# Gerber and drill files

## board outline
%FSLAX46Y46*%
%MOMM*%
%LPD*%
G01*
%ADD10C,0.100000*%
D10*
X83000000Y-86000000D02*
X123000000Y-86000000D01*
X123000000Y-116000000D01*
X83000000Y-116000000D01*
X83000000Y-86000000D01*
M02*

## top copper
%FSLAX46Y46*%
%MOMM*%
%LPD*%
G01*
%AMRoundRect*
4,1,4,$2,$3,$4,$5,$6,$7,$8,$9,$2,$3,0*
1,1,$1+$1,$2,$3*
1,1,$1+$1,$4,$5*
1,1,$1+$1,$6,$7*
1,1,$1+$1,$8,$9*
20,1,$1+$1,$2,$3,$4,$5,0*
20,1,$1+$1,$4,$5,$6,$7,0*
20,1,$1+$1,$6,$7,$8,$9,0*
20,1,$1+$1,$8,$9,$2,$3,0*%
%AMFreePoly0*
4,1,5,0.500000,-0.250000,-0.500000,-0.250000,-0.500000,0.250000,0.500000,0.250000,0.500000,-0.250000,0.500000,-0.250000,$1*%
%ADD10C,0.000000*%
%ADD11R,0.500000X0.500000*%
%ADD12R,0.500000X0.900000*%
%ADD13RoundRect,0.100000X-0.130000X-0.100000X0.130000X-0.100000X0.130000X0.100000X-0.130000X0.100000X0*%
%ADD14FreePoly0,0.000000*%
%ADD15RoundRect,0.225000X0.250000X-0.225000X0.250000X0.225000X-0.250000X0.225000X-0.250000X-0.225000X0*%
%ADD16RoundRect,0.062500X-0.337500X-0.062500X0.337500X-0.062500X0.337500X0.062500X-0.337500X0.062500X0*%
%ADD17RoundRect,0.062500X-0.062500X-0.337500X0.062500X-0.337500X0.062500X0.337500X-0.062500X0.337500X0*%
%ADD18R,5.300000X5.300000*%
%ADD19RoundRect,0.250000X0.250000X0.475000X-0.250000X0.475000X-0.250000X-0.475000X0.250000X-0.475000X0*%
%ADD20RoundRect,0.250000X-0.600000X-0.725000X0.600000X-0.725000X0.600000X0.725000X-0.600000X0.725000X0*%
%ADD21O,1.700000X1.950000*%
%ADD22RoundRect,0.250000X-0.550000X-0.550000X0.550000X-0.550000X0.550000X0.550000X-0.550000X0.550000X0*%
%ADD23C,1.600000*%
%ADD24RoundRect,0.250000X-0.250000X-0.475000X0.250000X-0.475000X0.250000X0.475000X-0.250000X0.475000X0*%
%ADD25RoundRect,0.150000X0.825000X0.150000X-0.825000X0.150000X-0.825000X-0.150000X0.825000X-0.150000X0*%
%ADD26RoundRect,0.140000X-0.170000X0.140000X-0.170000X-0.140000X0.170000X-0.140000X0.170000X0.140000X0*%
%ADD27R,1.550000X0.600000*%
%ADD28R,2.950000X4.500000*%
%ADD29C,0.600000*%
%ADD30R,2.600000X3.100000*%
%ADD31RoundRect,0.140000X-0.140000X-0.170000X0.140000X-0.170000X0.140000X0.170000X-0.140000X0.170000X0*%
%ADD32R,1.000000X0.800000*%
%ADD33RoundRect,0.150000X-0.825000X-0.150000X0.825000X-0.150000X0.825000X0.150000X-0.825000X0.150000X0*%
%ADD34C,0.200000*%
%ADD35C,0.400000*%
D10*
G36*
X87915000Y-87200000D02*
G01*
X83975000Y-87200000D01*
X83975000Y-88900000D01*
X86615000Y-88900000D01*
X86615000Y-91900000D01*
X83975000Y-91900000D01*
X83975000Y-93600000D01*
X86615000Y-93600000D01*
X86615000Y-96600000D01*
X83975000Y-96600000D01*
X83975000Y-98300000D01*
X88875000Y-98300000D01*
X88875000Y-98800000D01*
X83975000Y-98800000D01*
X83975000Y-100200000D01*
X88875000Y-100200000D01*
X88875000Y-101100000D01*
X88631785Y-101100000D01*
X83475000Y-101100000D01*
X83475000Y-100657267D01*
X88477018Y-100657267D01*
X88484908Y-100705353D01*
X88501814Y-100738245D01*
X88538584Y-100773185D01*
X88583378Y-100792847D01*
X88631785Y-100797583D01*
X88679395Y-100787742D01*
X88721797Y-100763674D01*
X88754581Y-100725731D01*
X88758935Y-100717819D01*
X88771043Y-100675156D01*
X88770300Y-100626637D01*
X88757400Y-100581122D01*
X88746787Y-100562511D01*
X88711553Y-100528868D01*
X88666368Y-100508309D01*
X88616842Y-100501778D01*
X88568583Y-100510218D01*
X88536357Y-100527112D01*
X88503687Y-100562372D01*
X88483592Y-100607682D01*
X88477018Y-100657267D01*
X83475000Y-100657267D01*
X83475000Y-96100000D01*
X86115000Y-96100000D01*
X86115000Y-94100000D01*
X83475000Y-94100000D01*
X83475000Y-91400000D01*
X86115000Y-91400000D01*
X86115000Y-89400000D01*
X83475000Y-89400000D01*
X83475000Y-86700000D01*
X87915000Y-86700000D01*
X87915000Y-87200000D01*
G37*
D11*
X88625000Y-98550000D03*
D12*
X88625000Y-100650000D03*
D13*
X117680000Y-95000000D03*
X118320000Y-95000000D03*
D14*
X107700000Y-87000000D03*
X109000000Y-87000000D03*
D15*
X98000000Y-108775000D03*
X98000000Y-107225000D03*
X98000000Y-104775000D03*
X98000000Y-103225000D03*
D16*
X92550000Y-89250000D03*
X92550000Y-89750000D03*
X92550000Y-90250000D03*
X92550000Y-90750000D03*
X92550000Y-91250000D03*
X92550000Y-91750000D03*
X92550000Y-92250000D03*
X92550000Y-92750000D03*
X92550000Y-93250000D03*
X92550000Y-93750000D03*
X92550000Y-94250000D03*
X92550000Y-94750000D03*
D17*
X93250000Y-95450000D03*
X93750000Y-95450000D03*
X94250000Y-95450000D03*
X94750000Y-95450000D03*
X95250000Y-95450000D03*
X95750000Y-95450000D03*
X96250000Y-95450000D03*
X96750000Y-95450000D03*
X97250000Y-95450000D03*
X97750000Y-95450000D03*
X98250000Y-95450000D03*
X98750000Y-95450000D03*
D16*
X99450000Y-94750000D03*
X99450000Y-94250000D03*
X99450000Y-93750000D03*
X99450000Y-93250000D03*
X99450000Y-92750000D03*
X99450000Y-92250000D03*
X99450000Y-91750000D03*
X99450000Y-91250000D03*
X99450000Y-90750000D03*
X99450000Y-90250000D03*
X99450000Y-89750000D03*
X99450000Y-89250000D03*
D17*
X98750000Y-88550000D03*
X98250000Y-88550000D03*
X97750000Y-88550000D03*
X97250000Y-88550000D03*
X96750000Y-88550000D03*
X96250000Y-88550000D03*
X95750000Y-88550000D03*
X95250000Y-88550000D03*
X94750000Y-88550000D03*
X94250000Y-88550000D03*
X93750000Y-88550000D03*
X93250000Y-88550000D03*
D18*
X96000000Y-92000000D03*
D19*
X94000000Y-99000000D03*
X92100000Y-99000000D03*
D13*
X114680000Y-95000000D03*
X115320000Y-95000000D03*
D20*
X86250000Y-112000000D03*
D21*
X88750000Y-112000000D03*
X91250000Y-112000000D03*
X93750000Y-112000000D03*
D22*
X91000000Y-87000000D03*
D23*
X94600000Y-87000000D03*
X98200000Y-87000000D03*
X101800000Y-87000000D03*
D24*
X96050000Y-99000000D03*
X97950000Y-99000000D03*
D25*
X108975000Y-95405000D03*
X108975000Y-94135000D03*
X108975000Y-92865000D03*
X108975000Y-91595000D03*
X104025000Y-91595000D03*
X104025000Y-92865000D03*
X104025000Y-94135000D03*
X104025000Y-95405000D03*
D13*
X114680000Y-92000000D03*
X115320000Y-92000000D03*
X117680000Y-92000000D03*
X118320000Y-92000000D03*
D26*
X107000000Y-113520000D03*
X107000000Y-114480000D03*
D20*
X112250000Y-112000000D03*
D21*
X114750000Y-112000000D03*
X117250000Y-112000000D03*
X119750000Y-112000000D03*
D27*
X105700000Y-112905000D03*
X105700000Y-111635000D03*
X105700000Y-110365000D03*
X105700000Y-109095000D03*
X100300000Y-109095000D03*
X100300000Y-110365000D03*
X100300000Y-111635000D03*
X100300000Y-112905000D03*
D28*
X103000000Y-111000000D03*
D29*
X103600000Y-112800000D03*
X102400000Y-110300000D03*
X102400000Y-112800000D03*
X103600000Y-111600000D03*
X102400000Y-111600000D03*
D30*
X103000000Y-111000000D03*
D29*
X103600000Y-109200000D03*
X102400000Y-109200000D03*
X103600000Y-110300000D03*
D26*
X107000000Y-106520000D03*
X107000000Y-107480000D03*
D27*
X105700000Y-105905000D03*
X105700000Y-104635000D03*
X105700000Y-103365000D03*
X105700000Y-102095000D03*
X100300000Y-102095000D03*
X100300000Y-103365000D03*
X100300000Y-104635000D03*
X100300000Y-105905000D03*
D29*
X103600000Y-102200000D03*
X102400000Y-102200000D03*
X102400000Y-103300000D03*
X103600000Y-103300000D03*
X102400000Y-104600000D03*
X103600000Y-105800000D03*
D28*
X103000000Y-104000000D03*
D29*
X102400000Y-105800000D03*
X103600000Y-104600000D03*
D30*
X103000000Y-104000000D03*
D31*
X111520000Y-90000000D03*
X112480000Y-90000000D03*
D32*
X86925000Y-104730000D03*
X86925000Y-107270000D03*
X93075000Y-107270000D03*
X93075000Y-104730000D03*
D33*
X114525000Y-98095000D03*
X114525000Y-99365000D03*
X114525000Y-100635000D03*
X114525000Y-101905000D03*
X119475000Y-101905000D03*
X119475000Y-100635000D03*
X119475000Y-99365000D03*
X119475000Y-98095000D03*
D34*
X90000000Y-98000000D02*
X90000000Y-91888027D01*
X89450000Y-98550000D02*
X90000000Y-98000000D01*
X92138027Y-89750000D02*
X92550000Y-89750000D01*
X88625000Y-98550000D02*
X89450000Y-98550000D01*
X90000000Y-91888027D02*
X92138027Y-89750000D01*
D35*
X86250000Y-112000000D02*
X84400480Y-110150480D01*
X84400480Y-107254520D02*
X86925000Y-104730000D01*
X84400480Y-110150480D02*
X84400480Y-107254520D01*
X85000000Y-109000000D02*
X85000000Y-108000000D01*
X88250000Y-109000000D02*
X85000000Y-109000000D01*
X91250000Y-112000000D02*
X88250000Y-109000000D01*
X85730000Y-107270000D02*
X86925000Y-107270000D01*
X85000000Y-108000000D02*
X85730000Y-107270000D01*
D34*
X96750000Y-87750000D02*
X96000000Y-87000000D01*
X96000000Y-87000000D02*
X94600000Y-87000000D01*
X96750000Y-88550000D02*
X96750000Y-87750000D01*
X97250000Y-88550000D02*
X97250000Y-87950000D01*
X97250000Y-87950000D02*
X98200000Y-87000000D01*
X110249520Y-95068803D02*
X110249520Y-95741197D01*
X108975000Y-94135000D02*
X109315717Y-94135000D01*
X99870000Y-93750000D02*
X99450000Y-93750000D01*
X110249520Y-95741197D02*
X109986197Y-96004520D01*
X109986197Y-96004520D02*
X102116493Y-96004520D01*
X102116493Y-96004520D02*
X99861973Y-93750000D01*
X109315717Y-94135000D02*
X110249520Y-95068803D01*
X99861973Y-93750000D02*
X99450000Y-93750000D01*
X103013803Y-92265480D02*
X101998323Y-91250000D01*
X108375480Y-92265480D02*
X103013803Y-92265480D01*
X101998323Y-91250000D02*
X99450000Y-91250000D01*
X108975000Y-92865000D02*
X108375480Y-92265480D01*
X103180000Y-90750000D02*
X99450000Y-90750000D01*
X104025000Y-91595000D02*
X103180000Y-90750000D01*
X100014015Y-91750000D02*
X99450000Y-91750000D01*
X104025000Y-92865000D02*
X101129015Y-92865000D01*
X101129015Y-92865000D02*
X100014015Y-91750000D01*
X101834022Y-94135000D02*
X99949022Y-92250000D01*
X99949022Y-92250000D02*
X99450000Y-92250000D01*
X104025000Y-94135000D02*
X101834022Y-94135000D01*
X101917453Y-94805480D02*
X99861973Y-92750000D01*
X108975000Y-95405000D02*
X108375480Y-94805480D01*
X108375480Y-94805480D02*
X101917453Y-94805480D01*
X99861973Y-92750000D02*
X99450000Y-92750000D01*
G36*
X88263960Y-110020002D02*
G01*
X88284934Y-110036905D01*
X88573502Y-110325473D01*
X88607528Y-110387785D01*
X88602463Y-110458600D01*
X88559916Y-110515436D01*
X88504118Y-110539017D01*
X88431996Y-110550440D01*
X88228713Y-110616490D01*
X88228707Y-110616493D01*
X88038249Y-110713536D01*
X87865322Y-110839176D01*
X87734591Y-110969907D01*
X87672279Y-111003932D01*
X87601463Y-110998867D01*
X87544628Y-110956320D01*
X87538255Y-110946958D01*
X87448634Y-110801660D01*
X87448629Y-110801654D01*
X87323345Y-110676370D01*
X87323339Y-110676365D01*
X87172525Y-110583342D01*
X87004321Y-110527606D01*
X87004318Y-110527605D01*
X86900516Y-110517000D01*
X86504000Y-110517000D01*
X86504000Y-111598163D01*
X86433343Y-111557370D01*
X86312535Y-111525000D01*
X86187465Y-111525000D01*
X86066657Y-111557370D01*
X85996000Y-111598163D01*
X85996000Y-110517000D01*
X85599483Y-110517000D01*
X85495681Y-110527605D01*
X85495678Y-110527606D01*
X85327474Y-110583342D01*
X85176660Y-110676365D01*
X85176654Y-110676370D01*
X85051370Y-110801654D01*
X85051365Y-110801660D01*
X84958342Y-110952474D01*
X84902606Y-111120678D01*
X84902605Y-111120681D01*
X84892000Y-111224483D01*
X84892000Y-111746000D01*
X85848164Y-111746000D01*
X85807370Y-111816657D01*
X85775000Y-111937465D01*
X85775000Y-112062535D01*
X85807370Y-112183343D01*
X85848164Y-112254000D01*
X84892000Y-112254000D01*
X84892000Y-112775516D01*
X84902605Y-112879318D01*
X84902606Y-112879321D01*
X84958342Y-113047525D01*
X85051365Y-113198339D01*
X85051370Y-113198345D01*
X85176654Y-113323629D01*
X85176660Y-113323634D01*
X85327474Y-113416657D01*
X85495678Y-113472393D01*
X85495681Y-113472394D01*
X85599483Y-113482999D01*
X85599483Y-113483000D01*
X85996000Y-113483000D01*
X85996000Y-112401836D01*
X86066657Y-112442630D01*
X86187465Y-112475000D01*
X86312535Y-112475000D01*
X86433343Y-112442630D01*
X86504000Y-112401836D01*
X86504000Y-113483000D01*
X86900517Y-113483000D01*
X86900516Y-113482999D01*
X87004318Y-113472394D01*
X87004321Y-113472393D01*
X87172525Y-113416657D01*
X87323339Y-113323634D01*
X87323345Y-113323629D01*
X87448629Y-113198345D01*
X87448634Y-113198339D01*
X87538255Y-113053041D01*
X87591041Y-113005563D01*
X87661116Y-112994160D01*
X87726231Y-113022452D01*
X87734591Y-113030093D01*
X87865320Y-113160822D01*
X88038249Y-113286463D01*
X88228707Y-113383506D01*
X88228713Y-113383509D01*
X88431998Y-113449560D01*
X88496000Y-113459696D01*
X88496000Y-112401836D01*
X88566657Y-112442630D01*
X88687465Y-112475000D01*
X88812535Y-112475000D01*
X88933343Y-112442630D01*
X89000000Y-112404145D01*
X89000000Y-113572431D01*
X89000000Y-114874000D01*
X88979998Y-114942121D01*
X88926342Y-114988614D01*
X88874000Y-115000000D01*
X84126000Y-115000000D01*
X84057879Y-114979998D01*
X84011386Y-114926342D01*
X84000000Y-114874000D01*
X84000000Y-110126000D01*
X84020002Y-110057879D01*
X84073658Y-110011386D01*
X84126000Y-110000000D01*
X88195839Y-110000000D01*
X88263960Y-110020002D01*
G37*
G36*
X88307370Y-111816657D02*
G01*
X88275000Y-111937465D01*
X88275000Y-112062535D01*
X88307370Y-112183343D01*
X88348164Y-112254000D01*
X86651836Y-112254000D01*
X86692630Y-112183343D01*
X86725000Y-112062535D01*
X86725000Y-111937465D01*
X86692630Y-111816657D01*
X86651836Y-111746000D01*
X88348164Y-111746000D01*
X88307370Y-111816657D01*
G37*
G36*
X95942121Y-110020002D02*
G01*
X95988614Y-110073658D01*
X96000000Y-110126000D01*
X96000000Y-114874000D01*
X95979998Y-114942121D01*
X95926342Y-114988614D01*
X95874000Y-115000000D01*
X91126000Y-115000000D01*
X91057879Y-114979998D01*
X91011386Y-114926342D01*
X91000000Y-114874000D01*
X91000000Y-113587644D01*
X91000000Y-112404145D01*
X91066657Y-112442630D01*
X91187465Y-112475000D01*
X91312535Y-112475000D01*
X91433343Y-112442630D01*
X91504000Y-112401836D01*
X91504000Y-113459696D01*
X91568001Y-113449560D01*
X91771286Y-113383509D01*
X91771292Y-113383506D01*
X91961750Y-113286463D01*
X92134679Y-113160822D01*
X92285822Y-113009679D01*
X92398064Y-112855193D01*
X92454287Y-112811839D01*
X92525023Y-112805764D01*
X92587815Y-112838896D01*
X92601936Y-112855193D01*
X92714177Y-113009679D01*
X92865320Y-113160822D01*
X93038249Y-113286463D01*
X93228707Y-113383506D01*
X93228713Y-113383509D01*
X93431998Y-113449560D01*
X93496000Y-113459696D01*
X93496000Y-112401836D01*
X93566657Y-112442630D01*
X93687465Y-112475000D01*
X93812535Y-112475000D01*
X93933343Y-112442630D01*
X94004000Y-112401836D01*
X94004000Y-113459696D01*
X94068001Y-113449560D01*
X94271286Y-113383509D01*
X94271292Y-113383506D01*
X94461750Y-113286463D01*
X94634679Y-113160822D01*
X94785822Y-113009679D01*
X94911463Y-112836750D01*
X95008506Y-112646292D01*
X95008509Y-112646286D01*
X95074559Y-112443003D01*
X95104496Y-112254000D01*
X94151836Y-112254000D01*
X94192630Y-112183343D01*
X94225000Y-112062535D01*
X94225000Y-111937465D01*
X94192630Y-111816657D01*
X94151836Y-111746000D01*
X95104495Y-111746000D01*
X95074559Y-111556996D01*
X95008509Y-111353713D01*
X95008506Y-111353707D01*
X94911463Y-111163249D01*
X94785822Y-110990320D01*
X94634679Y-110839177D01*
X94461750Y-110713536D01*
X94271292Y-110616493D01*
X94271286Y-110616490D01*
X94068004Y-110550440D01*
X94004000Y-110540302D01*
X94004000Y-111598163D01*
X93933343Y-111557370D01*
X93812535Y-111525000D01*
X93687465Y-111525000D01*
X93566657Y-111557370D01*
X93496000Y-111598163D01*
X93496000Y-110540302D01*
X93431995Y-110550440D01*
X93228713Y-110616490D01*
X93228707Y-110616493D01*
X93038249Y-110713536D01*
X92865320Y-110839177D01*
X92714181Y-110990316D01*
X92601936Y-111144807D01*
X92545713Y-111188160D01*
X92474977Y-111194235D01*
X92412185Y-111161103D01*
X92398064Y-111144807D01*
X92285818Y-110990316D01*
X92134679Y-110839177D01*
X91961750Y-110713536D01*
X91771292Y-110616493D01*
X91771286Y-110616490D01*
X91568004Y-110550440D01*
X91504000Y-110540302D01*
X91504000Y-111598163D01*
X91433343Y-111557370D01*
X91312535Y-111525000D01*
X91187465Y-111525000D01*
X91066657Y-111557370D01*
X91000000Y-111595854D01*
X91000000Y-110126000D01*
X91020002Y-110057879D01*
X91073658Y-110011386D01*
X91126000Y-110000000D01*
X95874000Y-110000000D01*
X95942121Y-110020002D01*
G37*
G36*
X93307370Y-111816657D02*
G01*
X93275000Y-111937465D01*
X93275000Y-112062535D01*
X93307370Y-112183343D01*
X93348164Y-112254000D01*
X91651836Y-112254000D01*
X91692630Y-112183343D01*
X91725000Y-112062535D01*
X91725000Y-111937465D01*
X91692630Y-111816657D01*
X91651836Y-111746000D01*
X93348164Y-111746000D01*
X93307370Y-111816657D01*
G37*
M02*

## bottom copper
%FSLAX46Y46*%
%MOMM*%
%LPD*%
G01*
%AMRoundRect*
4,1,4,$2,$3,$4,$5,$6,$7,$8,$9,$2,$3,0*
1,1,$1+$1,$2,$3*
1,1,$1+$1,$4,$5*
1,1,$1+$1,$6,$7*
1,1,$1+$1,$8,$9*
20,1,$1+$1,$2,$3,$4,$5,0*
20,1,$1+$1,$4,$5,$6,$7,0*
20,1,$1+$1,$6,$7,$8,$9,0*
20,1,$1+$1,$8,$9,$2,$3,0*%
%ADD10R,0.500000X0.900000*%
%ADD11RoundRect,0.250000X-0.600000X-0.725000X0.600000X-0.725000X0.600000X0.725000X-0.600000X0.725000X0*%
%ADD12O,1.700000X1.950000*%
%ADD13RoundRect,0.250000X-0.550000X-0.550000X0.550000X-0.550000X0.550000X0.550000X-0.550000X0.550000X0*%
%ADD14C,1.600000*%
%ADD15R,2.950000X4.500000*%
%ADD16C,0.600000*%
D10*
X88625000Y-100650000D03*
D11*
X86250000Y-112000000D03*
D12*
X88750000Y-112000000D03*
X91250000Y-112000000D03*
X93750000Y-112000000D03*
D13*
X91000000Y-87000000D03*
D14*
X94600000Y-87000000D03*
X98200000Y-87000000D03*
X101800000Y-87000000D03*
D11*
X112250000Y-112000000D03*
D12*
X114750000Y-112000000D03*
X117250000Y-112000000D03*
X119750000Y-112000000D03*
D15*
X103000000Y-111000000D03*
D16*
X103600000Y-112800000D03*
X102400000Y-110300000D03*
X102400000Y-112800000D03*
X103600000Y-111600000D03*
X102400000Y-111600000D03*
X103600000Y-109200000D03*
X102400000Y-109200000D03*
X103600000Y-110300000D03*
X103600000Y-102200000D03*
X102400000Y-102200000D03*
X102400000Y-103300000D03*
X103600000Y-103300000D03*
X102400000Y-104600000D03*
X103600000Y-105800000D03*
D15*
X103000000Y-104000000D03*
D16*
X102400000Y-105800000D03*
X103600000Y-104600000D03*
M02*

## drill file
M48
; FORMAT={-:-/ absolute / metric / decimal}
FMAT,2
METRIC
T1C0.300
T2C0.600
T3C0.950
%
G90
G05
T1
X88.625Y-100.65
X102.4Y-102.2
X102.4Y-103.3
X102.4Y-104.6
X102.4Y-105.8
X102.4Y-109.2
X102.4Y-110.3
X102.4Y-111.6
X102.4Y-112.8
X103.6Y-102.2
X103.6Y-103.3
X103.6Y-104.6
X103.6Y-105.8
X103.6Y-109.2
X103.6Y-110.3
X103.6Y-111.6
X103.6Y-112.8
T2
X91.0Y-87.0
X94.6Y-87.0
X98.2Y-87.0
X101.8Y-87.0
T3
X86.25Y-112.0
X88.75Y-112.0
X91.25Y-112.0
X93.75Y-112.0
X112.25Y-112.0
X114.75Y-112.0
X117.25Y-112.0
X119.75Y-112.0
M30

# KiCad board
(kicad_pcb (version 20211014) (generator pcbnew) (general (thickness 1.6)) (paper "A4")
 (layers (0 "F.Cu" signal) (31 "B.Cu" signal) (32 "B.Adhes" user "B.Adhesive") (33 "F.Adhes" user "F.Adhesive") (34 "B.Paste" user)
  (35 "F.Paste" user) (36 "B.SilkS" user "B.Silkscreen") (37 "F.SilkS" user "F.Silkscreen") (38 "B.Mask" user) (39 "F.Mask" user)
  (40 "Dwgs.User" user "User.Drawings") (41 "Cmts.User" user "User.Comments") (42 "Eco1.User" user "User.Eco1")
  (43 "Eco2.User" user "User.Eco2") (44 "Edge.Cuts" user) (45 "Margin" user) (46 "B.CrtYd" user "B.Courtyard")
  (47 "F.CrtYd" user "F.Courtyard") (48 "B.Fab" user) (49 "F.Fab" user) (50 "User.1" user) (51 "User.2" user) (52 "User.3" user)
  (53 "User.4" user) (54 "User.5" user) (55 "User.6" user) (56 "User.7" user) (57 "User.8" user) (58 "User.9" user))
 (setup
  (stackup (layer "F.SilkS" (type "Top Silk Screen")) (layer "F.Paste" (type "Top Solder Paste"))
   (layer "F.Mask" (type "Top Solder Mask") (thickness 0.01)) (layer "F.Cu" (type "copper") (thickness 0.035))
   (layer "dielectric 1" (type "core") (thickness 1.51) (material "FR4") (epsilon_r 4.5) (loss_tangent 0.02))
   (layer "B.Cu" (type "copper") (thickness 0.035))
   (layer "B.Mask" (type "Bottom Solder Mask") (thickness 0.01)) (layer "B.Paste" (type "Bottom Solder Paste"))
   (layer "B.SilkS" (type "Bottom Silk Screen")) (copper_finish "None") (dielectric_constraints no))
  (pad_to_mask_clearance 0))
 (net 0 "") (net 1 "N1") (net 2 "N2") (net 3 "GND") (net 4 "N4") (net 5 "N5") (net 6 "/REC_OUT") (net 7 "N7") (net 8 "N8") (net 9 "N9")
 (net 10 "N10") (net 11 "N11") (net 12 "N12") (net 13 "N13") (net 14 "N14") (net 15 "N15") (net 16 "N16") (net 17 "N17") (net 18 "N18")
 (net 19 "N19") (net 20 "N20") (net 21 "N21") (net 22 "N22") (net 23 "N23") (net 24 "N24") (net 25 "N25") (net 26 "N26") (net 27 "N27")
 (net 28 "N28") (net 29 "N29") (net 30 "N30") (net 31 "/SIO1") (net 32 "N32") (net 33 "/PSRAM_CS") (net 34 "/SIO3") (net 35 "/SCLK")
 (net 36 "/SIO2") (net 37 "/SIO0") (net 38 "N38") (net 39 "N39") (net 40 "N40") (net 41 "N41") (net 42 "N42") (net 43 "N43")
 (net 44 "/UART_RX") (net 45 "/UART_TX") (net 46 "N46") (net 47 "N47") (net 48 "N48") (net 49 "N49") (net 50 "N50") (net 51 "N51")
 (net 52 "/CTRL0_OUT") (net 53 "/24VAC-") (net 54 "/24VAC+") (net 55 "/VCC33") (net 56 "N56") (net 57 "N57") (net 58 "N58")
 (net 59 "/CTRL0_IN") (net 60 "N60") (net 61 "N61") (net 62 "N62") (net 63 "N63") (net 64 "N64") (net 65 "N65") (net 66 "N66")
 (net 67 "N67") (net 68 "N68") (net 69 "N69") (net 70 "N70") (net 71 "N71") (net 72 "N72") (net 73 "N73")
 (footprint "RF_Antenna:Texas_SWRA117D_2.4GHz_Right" (layer "F.Cu") (at 88.625 98.55 90)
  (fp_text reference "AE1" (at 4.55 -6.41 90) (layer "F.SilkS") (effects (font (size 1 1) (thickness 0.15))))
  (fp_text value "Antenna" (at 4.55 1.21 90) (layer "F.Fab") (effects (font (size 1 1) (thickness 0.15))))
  (fp_poly
   (pts (xy 2.45 -2.51) (xy 4.45 -2.51) (xy 4.45 -5.15) (xy 7.15 -5.15) (xy 7.15 -2.51) (xy 9.15 -2.51) (xy 9.15 -5.15) (xy 11.85 -5.15)
    (xy 11.85 -0.71) (xy 11.35 -0.71) (xy 11.35 -4.65) (xy 9.65 -4.65) (xy 9.65 -2.01) (xy 6.65 -2.01) (xy 6.65 -4.65) (xy 4.95 -4.65)
    (xy 4.95 -2.01) (xy 1.95 -2.01) (xy 1.95 -4.65) (xy 0.25 -4.65) (xy 0.25 0.25) (xy -0.25 0.25) (xy -0.25 -4.65) (xy -1.65 -4.65)
    (xy -1.65 0.25) (xy -2.55 0.25) (xy -2.55 0.006785) (xy -2.247583 0.006785) (xy -2.237742 0.054395) (xy -2.213674 0.096797)
    (xy -2.175731 0.129581) (xy -2.167819 0.133935) (xy -2.125156 0.146043) (xy -2.076637 0.1453) (xy -2.031122 0.1324)
    (xy -2.012511 0.121787) (xy -1.978868 0.086553) (xy -1.958309 0.041368) (xy -1.951778 -0.008158) (xy -1.960218 -0.056417)
    (xy -1.977112 -0.088643) (xy -2.012372 -0.121313) (xy -2.057682 -0.141408) (xy -2.107267 -0.147982) (xy -2.155353 -0.140092)
    (xy -2.188245 -0.123186) (xy -2.223185 -0.086416) (xy -2.242847 -0.041622) (xy -2.247583 0.006785) (xy -2.55 0.006785) (xy -2.55 -5.15)
    (xy 2.45 -5.15) (xy 2.45 -2.51))
   (layer "F.Cu") (width 0) (fill solid))
  (pad "1" connect rect (at 0 0 90) (size 0.5 0.5) (layers "F.Cu") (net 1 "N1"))
  (pad "2" thru_hole rect (at -2.1 0 90) (size 0.9 0.5) (drill 0.3) (layers *.Cu) (zone_connect 2)))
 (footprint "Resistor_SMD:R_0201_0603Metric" (layer "F.Cu") (at 118 95)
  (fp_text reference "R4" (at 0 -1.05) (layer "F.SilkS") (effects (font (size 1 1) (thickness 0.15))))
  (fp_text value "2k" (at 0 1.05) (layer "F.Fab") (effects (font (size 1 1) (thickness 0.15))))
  (pad "" smd roundrect (at 0.345 0) (size 0.318 0.36) (layers "F.Paste") (roundrect_rratio 0.25))
  (pad "" smd roundrect (at -0.345 0) (size 0.318 0.36) (layers "F.Paste") (roundrect_rratio 0.25))
  (pad "1" smd roundrect (at -0.32 0) (size 0.46 0.4) (layers "F.Cu" "F.Mask") (roundrect_rratio 0.25) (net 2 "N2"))
  (pad "2" smd roundrect (at 0.32 0) (size 0.46 0.4) (layers "F.Cu" "F.Mask") (roundrect_rratio 0.25) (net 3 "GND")))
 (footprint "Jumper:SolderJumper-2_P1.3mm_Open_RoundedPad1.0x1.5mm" (layer "F.Cu") (at 108.35 87)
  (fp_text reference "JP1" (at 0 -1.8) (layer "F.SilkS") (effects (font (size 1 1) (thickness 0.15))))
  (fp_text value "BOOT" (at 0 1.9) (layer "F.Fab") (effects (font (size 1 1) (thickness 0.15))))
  (pad "1" smd custom (at -0.65 0) (size 1 0.5) (layers "F.Cu" "F.Mask") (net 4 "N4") (zone_connect 2)
   (options (clearance outline) (anchor rect)) (primitives))
  (pad "2" smd custom (at 0.65 0) (size 1 0.5) (layers "F.Cu" "F.Mask") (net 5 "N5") (zone_connect 2)
   (options (clearance outline) (anchor rect)) (primitives)))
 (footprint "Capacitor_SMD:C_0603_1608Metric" (layer "F.Cu") (at 98 108 90)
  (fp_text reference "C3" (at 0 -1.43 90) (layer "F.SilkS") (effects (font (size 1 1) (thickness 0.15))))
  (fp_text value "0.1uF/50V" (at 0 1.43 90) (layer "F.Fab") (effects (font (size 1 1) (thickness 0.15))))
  (pad "1" smd roundrect (at -0.775 0 90) (size 0.9 0.95) (layers "F.Cu" "F.Paste" "F.Mask") (roundrect_rratio 0.25) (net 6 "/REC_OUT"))
  (pad "2" smd roundrect (at 0.775 0 90) (size 0.9 0.95) (layers "F.Cu" "F.Paste" "F.Mask") (roundrect_rratio 0.25) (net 3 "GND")))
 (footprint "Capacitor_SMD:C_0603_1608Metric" (layer "F.Cu") (at 98 104 90)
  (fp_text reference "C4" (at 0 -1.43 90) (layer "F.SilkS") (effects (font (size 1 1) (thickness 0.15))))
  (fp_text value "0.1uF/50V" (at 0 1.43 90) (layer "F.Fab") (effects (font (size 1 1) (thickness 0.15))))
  (pad "1" smd roundrect (at -0.775 0 90) (size 0.9 0.95) (layers "F.Cu" "F.Paste" "F.Mask") (roundrect_rratio 0.25) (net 6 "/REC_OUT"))
  (pad "2" smd roundrect (at 0.775 0 90) (size 0.9 0.95) (layers "F.Cu" "F.Paste" "F.Mask") (roundrect_rratio 0.25) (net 3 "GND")))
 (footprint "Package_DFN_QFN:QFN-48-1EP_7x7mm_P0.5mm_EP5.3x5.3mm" (layer "F.Cu") (at 96 92)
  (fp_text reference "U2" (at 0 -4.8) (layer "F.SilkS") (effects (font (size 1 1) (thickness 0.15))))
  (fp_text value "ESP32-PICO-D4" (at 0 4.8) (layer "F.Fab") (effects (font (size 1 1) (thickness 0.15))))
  (pad "" smd roundrect (at -1.98 -0.66) (size 1.07 1.07) (layers "F.Paste") (roundrect_rratio 0.233645))
  (pad "" smd roundrect (at 0.66 1.98) (size 1.07 1.07) (layers "F.Paste") (roundrect_rratio 0.233645))
  (pad "" smd roundrect (at 1.98 0.66) (size 1.07 1.07) (layers "F.Paste") (roundrect_rratio 0.233645))
  (pad "" smd roundrect (at -0.66 0.66) (size 1.07 1.07) (layers "F.Paste") (roundrect_rratio 0.233645))
  (pad "" smd roundrect (at 0.66 0.66) (size 1.07 1.07) (layers "F.Paste") (roundrect_rratio 0.233645))
  (pad "" smd roundrect (at -1.98 -1.98) (size 1.07 1.07) (layers "F.Paste") (roundrect_rratio 0.233645))
  (pad "" smd roundrect (at -0.66 -1.98) (size 1.07 1.07) (layers "F.Paste") (roundrect_rratio 0.233645))
  (pad "" smd roundrect (at 1.98 1.98) (size 1.07 1.07) (layers "F.Paste") (roundrect_rratio 0.233645))
  (pad "" smd roundrect (at -1.98 1.98) (size 1.07 1.07) (layers "F.Paste") (roundrect_rratio 0.233645))
  (pad "" smd roundrect (at 1.98 -1.98) (size 1.07 1.07) (layers "F.Paste") (roundrect_rratio 0.233645))
  (pad "" smd roundrect (at -1.98 0.66) (size 1.07 1.07) (layers "F.Paste") (roundrect_rratio 0.233645))
  (pad "" smd roundrect (at 0.66 -1.98) (size 1.07 1.07) (layers "F.Paste") (roundrect_rratio 0.233645))
  (pad "" smd roundrect (at -0.66 1.98) (size 1.07 1.07) (layers "F.Paste") (roundrect_rratio 0.233645))
  (pad "" smd roundrect (at 1.98 -0.66) (size 1.07 1.07) (layers "F.Paste") (roundrect_rratio 0.233645))
  (pad "" smd roundrect (at -0.66 -0.66) (size 1.07 1.07) (layers "F.Paste") (roundrect_rratio 0.233645))
  (pad "" smd roundrect (at 0.66 -0.66) (size 1.07 1.07) (layers "F.Paste") (roundrect_rratio 0.233645))
  (pad "1" smd roundrect (at -3.45 -2.75) (size 0.8 0.25) (layers "F.Cu" "F.Paste" "F.Mask") (roundrect_rratio 0.25) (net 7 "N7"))
  (pad "2" smd roundrect (at -3.45 -2.25) (size 0.8 0.25) (layers "F.Cu" "F.Paste" "F.Mask") (roundrect_rratio 0.25) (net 1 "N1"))
  (pad "3" smd roundrect (at -3.45 -1.75) (size 0.8 0.25) (layers "F.Cu" "F.Paste" "F.Mask") (roundrect_rratio 0.25) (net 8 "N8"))
  (pad "4" smd roundrect (at -3.45 -1.25) (size 0.8 0.25) (layers "F.Cu" "F.Paste" "F.Mask") (roundrect_rratio 0.25) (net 8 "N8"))
  (pad "5" smd roundrect (at -3.45 -0.75) (size 0.8 0.25) (layers "F.Cu" "F.Paste" "F.Mask") (roundrect_rratio 0.25) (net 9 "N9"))
  (pad "6" smd roundrect (at -3.45 -0.25) (size 0.8 0.25) (layers "F.Cu" "F.Paste" "F.Mask") (roundrect_rratio 0.25) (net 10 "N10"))
  (pad "7" smd roundrect (at -3.45 0.25) (size 0.8 0.25) (layers "F.Cu" "F.Paste" "F.Mask") (roundrect_rratio 0.25) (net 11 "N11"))
  (pad "8" smd roundrect (at -3.45 0.75) (size 0.8 0.25) (layers "F.Cu" "F.Paste" "F.Mask") (roundrect_rratio 0.25) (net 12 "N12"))
  (pad "9" smd roundrect (at -3.45 1.25) (size 0.8 0.25) (layers "F.Cu" "F.Paste" "F.Mask") (roundrect_rratio 0.25) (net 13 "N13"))
  (pad "10" smd roundrect (at -3.45 1.75) (size 0.8 0.25) (layers "F.Cu" "F.Paste" "F.Mask") (roundrect_rratio 0.25) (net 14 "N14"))
  (pad "11" smd roundrect (at -3.45 2.25) (size 0.8 0.25) (layers "F.Cu" "F.Paste" "F.Mask") (roundrect_rratio 0.25) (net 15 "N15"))
  (pad "12" smd roundrect (at -3.45 2.75) (size 0.8 0.25) (layers "F.Cu" "F.Paste" "F.Mask") (roundrect_rratio 0.25) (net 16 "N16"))
  (pad "13" smd roundrect (at -2.75 3.45) (size 0.25 0.8) (layers "F.Cu" "F.Paste" "F.Mask") (roundrect_rratio 0.25) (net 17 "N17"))
  (pad "14" smd roundrect (at -2.25 3.45) (size 0.25 0.8) (layers "F.Cu" "F.Paste" "F.Mask") (roundrect_rratio 0.25) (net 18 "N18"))
  (pad "15" smd roundrect (at -1.75 3.45) (size 0.25 0.8) (layers "F.Cu" "F.Paste" "F.Mask") (roundrect_rratio 0.25) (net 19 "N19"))
  (pad "16" smd roundrect (at -1.25 3.45) (size 0.25 0.8) (layers "F.Cu" "F.Paste" "F.Mask") (roundrect_rratio 0.25) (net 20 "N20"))
  (pad "17" smd roundrect (at -0.75 3.45) (size 0.25 0.8) (layers "F.Cu" "F.Paste" "F.Mask") (roundrect_rratio 0.25) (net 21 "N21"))
  (pad "18" smd roundrect (at -0.25 3.45) (size 0.25 0.8) (layers "F.Cu" "F.Paste" "F.Mask") (roundrect_rratio 0.25) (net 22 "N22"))
  (pad "19" smd roundrect (at 0.25 3.45) (size 0.25 0.8) (layers "F.Cu" "F.Paste" "F.Mask") (roundrect_rratio 0.25) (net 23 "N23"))
  (pad "20" smd roundrect (at 0.75 3.45) (size 0.25 0.8) (layers "F.Cu" "F.Paste" "F.Mask") (roundrect_rratio 0.25) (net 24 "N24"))
  (pad "21" smd roundrect (at 1.25 3.45) (size 0.25 0.8) (layers "F.Cu" "F.Paste" "F.Mask") (roundrect_rratio 0.25) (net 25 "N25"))
  (pad "22" smd roundrect (at 1.75 3.45) (size 0.25 0.8) (layers "F.Cu" "F.Paste" "F.Mask") (roundrect_rratio 0.25) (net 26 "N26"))
  (pad "23" smd roundrect (at 2.25 3.45) (size 0.25 0.8) (layers "F.Cu" "F.Paste" "F.Mask") (roundrect_rratio 0.25) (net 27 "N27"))
  (pad "24" smd roundrect (at 2.75 3.45) (size 0.25 0.8) (layers "F.Cu" "F.Paste" "F.Mask") (roundrect_rratio 0.25) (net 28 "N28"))
  (pad "25" smd roundrect (at 3.45 2.75) (size 0.8 0.25) (layers "F.Cu" "F.Paste" "F.Mask") (roundrect_rratio 0.25) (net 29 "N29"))
  (pad "26" smd roundrect (at 3.45 2.25) (size 0.8 0.25) (layers "F.Cu" "F.Paste" "F.Mask") (roundrect_rratio 0.25) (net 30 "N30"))
  (pad "27" smd roundrect (at 3.45 1.75) (size 0.8 0.25) (layers "F.Cu" "F.Paste" "F.Mask") (roundrect_rratio 0.25) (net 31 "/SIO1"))
  (pad "28" smd roundrect (at 3.45 1.25) (size 0.8 0.25) (layers "F.Cu" "F.Paste" "F.Mask") (roundrect_rratio 0.25) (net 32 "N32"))
  (pad "29" smd roundrect (at 3.45 0.75) (size 0.8 0.25) (layers "F.Cu" "F.Paste" "F.Mask") (roundrect_rratio 0.25) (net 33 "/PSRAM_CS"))
  (pad "30" smd roundrect (at 3.45 0.25) (size 0.8 0.25) (layers "F.Cu" "F.Paste" "F.Mask") (roundrect_rratio 0.25) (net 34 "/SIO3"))
  (pad "31" smd roundrect (at 3.45 -0.25) (size 0.8 0.25) (layers "F.Cu" "F.Paste" "F.Mask") (roundrect_rratio 0.25) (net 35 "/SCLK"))
  (pad "32" smd roundrect (at 3.45 -0.75) (size 0.8 0.25) (layers "F.Cu" "F.Paste" "F.Mask") (roundrect_rratio 0.25) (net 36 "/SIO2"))
  (pad "33" smd roundrect (at 3.45 -1.25) (size 0.8 0.25) (layers "F.Cu" "F.Paste" "F.Mask") (roundrect_rratio 0.25) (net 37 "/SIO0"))
  (pad "34" smd roundrect (at 3.45 -1.75) (size 0.8 0.25) (layers "F.Cu" "F.Paste" "F.Mask") (roundrect_rratio 0.25) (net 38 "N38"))
  (pad "35" smd roundrect (at 3.45 -2.25) (size 0.8 0.25) (layers "F.Cu" "F.Paste" "F.Mask") (roundrect_rratio 0.25) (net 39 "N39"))
  (pad "36" smd roundrect (at 3.45 -2.75) (size 0.8 0.25) (layers "F.Cu" "F.Paste" "F.Mask") (roundrect_rratio 0.25) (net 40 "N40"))
  (pad "37" smd roundrect (at 2.75 -3.45) (size 0.25 0.8) (layers "F.Cu" "F.Paste" "F.Mask") (roundrect_rratio 0.25) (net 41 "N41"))
  (pad "38" smd roundrect (at 2.25 -3.45) (size 0.25 0.8) (layers "F.Cu" "F.Paste" "F.Mask") (roundrect_rratio 0.25) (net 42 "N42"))
  (pad "39" smd roundrect (at 1.75 -3.45) (size 0.25 0.8) (layers "F.Cu" "F.Paste" "F.Mask") (roundrect_rratio 0.25) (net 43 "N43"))
  (pad "40" smd roundrect (at 1.25 -3.45) (size 0.25 0.8) (layers "F.Cu" "F.Paste" "F.Mask") (roundrect_rratio 0.25) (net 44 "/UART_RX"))
  (pad "41" smd roundrect (at 0.75 -3.45) (size 0.25 0.8) (layers "F.Cu" "F.Paste" "F.Mask") (roundrect_rratio 0.25) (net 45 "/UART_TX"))
  (pad "42" smd roundrect (at 0.25 -3.45) (size 0.25 0.8) (layers "F.Cu" "F.Paste" "F.Mask") (roundrect_rratio 0.25) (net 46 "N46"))
  (pad "43" smd roundrect (at -0.25 -3.45) (size 0.25 0.8) (layers "F.Cu" "F.Paste" "F.Mask") (roundrect_rratio 0.25) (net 7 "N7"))
  (pad "44" smd roundrect (at -0.75 -3.45) (size 0.25 0.8) (layers "F.Cu" "F.Paste" "F.Mask") (roundrect_rratio 0.25) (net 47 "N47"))
  (pad "45" smd roundrect (at -1.25 -3.45) (size 0.25 0.8) (layers "F.Cu" "F.Paste" "F.Mask") (roundrect_rratio 0.25) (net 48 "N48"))
  (pad "46" smd roundrect (at -1.75 -3.45) (size 0.25 0.8) (layers "F.Cu" "F.Paste" "F.Mask") (roundrect_rratio 0.25) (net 7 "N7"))
  (pad "47" smd roundrect (at -2.25 -3.45) (size 0.25 0.8) (layers "F.Cu" "F.Paste" "F.Mask") (roundrect_rratio 0.25) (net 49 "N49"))
  (pad "48" smd roundrect (at -2.75 -3.45) (size 0.25 0.8) (layers "F.Cu" "F.Paste" "F.Mask") (roundrect_rratio 0.25) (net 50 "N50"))
  (pad "49" smd rect (at 0 0) (size 5.3 5.3) (layers "F.Cu" "F.Mask") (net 3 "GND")))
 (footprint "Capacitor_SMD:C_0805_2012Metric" (layer "F.Cu") (at 93.05 99 180)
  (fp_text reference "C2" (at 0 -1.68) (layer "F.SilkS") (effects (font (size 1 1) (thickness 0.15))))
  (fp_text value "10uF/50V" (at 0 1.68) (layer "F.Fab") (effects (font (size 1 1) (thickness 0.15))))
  (pad "1" smd roundrect (at -0.95 0 180) (size 1 1.45) (layers "F.Cu" "F.Paste" "F.Mask") (roundrect_rratio 0.25) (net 6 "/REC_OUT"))
  (pad "2" smd roundrect (at 0.95 0 180) (size 1 1.45) (layers "F.Cu" "F.Paste" "F.Mask") (roundrect_rratio 0.25) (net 3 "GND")))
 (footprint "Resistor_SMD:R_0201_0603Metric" (layer "F.Cu") (at 115 95)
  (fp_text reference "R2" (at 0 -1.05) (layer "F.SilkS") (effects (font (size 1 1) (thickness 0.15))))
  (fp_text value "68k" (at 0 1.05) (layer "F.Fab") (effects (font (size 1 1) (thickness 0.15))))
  (pad "" smd roundrect (at 0.345 0) (size 0.318 0.36) (layers "F.Paste") (roundrect_rratio 0.25))
  (pad "" smd roundrect (at -0.345 0) (size 0.318 0.36) (layers "F.Paste") (roundrect_rratio 0.25))
  (pad "1" smd roundrect (at -0.32 0) (size 0.46 0.4) (layers "F.Cu" "F.Mask") (roundrect_rratio 0.25) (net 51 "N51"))
  (pad "2" smd roundrect (at 0.32 0) (size 0.46 0.4) (layers "F.Cu" "F.Mask") (roundrect_rratio 0.25) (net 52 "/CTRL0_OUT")))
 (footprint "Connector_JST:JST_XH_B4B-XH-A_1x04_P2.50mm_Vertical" (layer "F.Cu") (at 86.25 112)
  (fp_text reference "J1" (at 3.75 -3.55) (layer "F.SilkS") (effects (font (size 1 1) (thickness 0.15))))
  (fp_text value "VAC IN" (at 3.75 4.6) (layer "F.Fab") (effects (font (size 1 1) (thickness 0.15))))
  (pad "1" thru_hole roundrect (at 0 0) (size 1.7 1.95) (drill 0.95) (layers *.Cu *.Mask) (roundrect_rratio 0.147059) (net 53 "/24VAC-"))
  (pad "2" thru_hole oval (at 2.5 0) (size 1.7 1.95) (drill 0.95) (layers *.Cu *.Mask) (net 53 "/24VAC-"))
  (pad "3" thru_hole oval (at 5 0) (size 1.7 1.95) (drill 0.95) (layers *.Cu *.Mask) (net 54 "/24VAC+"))
  (pad "4" thru_hole oval (at 7.5 0) (size 1.7 1.95) (drill 0.95) (layers *.Cu *.Mask) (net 54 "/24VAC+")))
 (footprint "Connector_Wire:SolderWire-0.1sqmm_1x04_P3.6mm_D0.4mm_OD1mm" (layer "F.Cu") (at 91 87)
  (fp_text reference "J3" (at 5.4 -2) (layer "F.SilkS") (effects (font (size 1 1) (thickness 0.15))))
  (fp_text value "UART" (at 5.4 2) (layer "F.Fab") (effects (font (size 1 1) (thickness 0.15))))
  (pad "1" thru_hole roundrect (at 0 0) (size 1.6 1.6) (drill 0.6) (layers *.Cu *.Mask) (roundrect_rratio 0.15625) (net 3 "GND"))
  (pad "2" thru_hole circle (at 3.6 0) (size 1.6 1.6) (drill 0.6) (layers *.Cu *.Mask) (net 45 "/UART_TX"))
  (pad "3" thru_hole circle (at 7.2 0) (size 1.6 1.6) (drill 0.6) (layers *.Cu *.Mask) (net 44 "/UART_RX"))
  (pad "4" thru_hole circle (at 10.8 0) (size 1.6 1.6) (drill 0.6) (layers *.Cu *.Mask) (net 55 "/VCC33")))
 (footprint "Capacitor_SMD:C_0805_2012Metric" (layer "F.Cu") (at 97 99)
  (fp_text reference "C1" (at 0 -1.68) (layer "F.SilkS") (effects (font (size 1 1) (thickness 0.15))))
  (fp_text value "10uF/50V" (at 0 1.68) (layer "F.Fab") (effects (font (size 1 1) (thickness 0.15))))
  (pad "1" smd roundrect (at -0.95 0) (size 1 1.45) (layers "F.Cu" "F.Paste" "F.Mask") (roundrect_rratio 0.25) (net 6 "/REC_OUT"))
  (pad "2" smd roundrect (at 0.95 0) (size 1 1.45) (layers "F.Cu" "F.Paste" "F.Mask") (roundrect_rratio 0.25) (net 3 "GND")))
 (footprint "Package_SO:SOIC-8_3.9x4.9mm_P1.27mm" (layer "F.Cu") (at 106.5 93.5 180)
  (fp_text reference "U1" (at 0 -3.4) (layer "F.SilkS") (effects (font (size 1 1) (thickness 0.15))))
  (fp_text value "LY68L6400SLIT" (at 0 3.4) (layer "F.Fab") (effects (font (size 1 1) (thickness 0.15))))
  (pad "1" smd roundrect (at -2.475 -1.905 180) (size 1.95 0.6) (layers "F.Cu" "F.Paste" "F.Mask") (roundrect_rratio 0.25)
   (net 33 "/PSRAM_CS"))
  (pad "2" smd roundrect (at -2.475 -0.635 180) (size 1.95 0.6) (layers "F.Cu" "F.Paste" "F.Mask") (roundrect_rratio 0.25) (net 31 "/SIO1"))
  (pad "3" smd roundrect (at -2.475 0.635 180) (size 1.95 0.6) (layers "F.Cu" "F.Paste" "F.Mask") (roundrect_rratio 0.25) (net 36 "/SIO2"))
  (pad "4" smd roundrect (at -2.475 1.905 180) (size 1.95 0.6) (layers "F.Cu" "F.Paste" "F.Mask") (roundrect_rratio 0.25) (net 3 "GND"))
  (pad "5" smd roundrect (at 2.475 1.905 180) (size 1.95 0.6) (layers "F.Cu" "F.Paste" "F.Mask") (roundrect_rratio 0.25) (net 37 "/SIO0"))
  (pad "6" smd roundrect (at 2.475 0.635 180) (size 1.95 0.6) (layers "F.Cu" "F.Paste" "F.Mask") (roundrect_rratio 0.25) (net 35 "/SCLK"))
  (pad "7" smd roundrect (at 2.475 -0.635 180) (size 1.95 0.6) (layers "F.Cu" "F.Paste" "F.Mask") (roundrect_rratio 0.25) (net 34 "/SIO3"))
  (pad "8" smd roundrect (at 2.475 -1.905 180) (size 1.95 0.6) (layers "F.Cu" "F.Paste" "F.Mask") (roundrect_rratio 0.25) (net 55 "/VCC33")))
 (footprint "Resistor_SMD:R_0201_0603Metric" (layer "F.Cu") (at 115 92)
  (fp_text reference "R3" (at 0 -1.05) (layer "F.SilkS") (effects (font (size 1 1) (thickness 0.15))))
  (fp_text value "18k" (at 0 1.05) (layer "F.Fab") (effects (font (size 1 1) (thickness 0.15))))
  (pad "" smd roundrect (at 0.345 0) (size 0.318 0.36) (layers "F.Paste") (roundrect_rratio 0.25))
  (pad "" smd roundrect (at -0.345 0) (size 0.318 0.36) (layers "F.Paste") (roundrect_rratio 0.25))
  (pad "1" smd roundrect (at -0.32 0) (size 0.46 0.4) (layers "F.Cu" "F.Mask") (roundrect_rratio 0.25) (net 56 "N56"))
  (pad "2" smd roundrect (at 0.32 0) (size 0.46 0.4) (layers "F.Cu" "F.Mask") (roundrect_rratio 0.25) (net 2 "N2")))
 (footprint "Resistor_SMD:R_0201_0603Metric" (layer "F.Cu") (at 118 92)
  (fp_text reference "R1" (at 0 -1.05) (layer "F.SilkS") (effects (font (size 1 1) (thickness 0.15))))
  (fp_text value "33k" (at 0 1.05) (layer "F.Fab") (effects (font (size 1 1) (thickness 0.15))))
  (pad "" smd roundrect (at 0.345 0) (size 0.318 0.36) (layers "F.Paste") (roundrect_rratio 0.25))
  (pad "" smd roundrect (at -0.345 0) (size 0.318 0.36) (layers "F.Paste") (roundrect_rratio 0.25))
  (pad "1" smd roundrect (at -0.32 0) (size 0.46 0.4) (layers "F.Cu" "F.Mask") (roundrect_rratio 0.25) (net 51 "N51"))
  (pad "2" smd roundrect (at 0.32 0) (size 0.46 0.4) (layers "F.Cu" "F.Mask") (roundrect_rratio 0.25) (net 3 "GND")))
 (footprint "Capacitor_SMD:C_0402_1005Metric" (layer "F.Cu") (at 107 114 -90)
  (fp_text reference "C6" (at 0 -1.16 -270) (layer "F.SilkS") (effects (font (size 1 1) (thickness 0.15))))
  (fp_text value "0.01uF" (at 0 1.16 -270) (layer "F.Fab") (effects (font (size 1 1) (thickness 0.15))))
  (pad "1" smd roundrect (at -0.48 0 270) (size 0.56 0.62) (layers "F.Cu" "F.Paste" "F.Mask") (roundrect_rratio 0.25) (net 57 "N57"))
  (pad "2" smd roundrect (at 0.48 0 270) (size 0.56 0.62) (layers "F.Cu" "F.Paste" "F.Mask") (roundrect_rratio 0.25) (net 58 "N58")))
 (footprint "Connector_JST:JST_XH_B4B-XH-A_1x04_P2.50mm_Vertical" (layer "F.Cu") (at 112.25 112)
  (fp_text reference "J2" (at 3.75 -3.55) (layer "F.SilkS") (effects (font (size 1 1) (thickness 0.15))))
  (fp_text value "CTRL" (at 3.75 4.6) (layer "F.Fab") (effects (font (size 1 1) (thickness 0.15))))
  (pad "1" thru_hole roundrect (at 0 0) (size 1.7 1.95) (drill 0.95) (layers *.Cu *.Mask) (roundrect_rratio 0.147059) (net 3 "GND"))
  (pad "2" thru_hole oval (at 2.5 0) (size 1.7 1.95) (drill 0.95) (layers *.Cu *.Mask) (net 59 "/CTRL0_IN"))
  (pad "3" thru_hole oval (at 5 0) (size 1.7 1.95) (drill 0.95) (layers *.Cu *.Mask) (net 52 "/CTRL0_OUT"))
  (pad "4" thru_hole oval (at 7.5 0) (size 1.7 1.95) (drill 0.95) (layers *.Cu *.Mask) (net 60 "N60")))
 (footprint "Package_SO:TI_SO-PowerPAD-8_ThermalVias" (layer "F.Cu") (at 103 111 180)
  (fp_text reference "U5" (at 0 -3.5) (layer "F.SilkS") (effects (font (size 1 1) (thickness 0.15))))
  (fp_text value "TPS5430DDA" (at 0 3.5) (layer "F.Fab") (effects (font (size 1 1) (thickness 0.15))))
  (pad "1" smd rect (at -2.7 -1.905 180) (size 1.55 0.6) (layers "F.Cu" "F.Paste" "F.Mask") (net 57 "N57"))
  (pad "2" smd rect (at -2.7 -0.635 180) (size 1.55 0.6) (layers "F.Cu" "F.Paste" "F.Mask") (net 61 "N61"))
  (pad "3" smd rect (at -2.7 0.635 180) (size 1.55 0.6) (layers "F.Cu" "F.Paste" "F.Mask") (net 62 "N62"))
  (pad "4" smd rect (at -2.7 1.905 180) (size 1.55 0.6) (layers "F.Cu" "F.Paste" "F.Mask") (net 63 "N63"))
  (pad "5" smd rect (at 2.7 1.905 180) (size 1.55 0.6) (layers "F.Cu" "F.Paste" "F.Mask") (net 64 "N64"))
  (pad "6" smd rect (at 2.7 0.635 180) (size 1.55 0.6) (layers "F.Cu" "F.Paste" "F.Mask") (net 3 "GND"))
  (pad "7" smd rect (at 2.7 -0.635 180) (size 1.55 0.6) (layers "F.Cu" "F.Paste" "F.Mask") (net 6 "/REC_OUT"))
  (pad "8" smd rect (at 2.7 -1.905 180) (size 1.55 0.6) (layers "F.Cu" "F.Paste" "F.Mask") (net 58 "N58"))
  (pad "9" smd rect (at 0 0 180) (size 2.95 4.5) (layers "F.Cu") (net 3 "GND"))
  (pad "9" smd rect (at 0 0 180) (size 2.95 4.5) (layers "B.Cu") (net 3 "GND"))
  (pad "9" thru_hole circle (at -0.6 -1.8 180) (size 0.6 0.6) (drill 0.3) (layers *.Cu) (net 3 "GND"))
  (pad "9" thru_hole circle (at 0.6 0.7 180) (size 0.6 0.6) (drill 0.3) (layers *.Cu) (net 3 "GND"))
  (pad "9" thru_hole circle (at 0.6 -1.8 180) (size 0.6 0.6) (drill 0.3) (layers *.Cu) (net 3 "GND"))
  (pad "9" thru_hole circle (at -0.6 -0.6 180) (size 0.6 0.6) (drill 0.3) (layers *.Cu) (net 3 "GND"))
  (pad "9" thru_hole circle (at 0.6 -0.6 180) (size 0.6 0.6) (drill 0.3) (layers *.Cu) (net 3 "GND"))
  (pad "9" smd rect (at 0 0 180) (size 2.6 3.1) (layers "F.Cu" "F.Paste" "F.Mask") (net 3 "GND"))
  (pad "9" thru_hole circle (at -0.6 1.8 180) (size 0.6 0.6) (drill 0.3) (layers *.Cu) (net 3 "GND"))
  (pad "9" thru_hole circle (at 0.6 1.8 180) (size 0.6 0.6) (drill 0.3) (layers *.Cu) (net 3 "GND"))
  (pad "9" thru_hole circle (at -0.6 0.7 180) (size 0.6 0.6) (drill 0.3) (layers *.Cu) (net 3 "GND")))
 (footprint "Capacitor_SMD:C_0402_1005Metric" (layer "F.Cu") (at 107 107 -90)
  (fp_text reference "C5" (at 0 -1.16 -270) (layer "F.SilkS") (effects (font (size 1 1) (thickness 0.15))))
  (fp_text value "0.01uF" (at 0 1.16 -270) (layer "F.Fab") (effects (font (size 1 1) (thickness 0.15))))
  (pad "1" smd roundrect (at -0.48 0 270) (size 0.56 0.62) (layers "F.Cu" "F.Paste" "F.Mask") (roundrect_rratio 0.25) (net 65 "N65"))
  (pad "2" smd roundrect (at 0.48 0 270) (size 0.56 0.62) (layers "F.Cu" "F.Paste" "F.Mask") (roundrect_rratio 0.25) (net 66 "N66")))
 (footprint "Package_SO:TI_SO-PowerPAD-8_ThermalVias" (layer "F.Cu") (at 103 104 180)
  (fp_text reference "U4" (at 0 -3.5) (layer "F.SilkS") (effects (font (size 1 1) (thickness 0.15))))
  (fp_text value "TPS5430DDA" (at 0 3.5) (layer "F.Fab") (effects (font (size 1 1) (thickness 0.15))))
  (pad "1" smd rect (at -2.7 -1.905 180) (size 1.55 0.6) (layers "F.Cu" "F.Paste" "F.Mask") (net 65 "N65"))
  (pad "2" smd rect (at -2.7 -0.635 180) (size 1.55 0.6) (layers "F.Cu" "F.Paste" "F.Mask") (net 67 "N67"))
  (pad "3" smd rect (at -2.7 0.635 180) (size 1.55 0.6) (layers "F.Cu" "F.Paste" "F.Mask") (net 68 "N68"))
  (pad "4" smd rect (at -2.7 1.905 180) (size 1.55 0.6) (layers "F.Cu" "F.Paste" "F.Mask") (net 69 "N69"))
  (pad "5" smd rect (at 2.7 1.905 180) (size 1.55 0.6) (layers "F.Cu" "F.Paste" "F.Mask") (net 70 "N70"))
  (pad "6" smd rect (at 2.7 0.635 180) (size 1.55 0.6) (layers "F.Cu" "F.Paste" "F.Mask") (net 3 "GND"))
  (pad "7" smd rect (at 2.7 -0.635 180) (size 1.55 0.6) (layers "F.Cu" "F.Paste" "F.Mask") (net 6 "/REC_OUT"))
  (pad "8" smd rect (at 2.7 -1.905 180) (size 1.55 0.6) (layers "F.Cu" "F.Paste" "F.Mask") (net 66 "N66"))
  (pad "9" thru_hole circle (at -0.6 1.8 180) (size 0.6 0.6) (drill 0.3) (layers *.Cu) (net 3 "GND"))
  (pad "9" thru_hole circle (at 0.6 1.8 180) (size 0.6 0.6) (drill 0.3) (layers *.Cu) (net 3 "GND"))
  (pad "9" thru_hole circle (at 0.6 0.7 180) (size 0.6 0.6) (drill 0.3) (layers *.Cu) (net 3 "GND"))
  (pad "9" thru_hole circle (at -0.6 0.7 180) (size 0.6 0.6) (drill 0.3) (layers *.Cu) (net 3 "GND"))
  (pad "9" thru_hole circle (at 0.6 -0.6 180) (size 0.6 0.6) (drill 0.3) (layers *.Cu) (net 3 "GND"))
  (pad "9" thru_hole circle (at -0.6 -1.8 180) (size 0.6 0.6) (drill 0.3) (layers *.Cu) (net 3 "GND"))
  (pad "9" smd rect (at 0 0 180) (size 2.95 4.5) (layers "F.Cu") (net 3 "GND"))
  (pad "9" smd rect (at 0 0 180) (size 2.95 4.5) (layers "B.Cu") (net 3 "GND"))
  (pad "9" thru_hole circle (at 0.6 -1.8 180) (size 0.6 0.6) (drill 0.3) (layers *.Cu) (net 3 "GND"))
  (pad "9" thru_hole circle (at -0.6 -0.6 180) (size 0.6 0.6) (drill 0.3) (layers *.Cu) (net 3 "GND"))
  (pad "9" smd rect (at 0 0 180) (size 2.6 3.1) (layers "F.Cu" "F.Paste" "F.Mask") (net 3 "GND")))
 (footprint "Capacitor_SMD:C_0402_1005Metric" (layer "F.Cu") (at 112 90)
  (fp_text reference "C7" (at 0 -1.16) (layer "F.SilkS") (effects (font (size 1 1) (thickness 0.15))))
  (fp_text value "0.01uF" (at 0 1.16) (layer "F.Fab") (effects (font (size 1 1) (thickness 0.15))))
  (pad "1" smd roundrect (at -0.48 0) (size 0.56 0.62) (layers "F.Cu" "F.Paste" "F.Mask") (roundrect_rratio 0.25) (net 55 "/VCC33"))
  (pad "2" smd roundrect (at 0.48 0) (size 0.56 0.62) (layers "F.Cu" "F.Paste" "F.Mask") (roundrect_rratio 0.25) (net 3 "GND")))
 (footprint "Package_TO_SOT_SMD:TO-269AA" (layer "F.Cu") (at 90 106)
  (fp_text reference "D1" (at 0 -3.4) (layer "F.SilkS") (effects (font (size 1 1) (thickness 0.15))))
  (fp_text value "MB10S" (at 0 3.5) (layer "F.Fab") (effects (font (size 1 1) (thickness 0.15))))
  (pad "1" smd rect (at -3.075 -1.27) (size 1 0.8) (layers "F.Cu" "F.Paste" "F.Mask") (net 53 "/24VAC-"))
  (pad "2" smd rect (at -3.075 1.27) (size 1 0.8) (layers "F.Cu" "F.Paste" "F.Mask") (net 54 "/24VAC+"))
  (pad "3" smd rect (at 3.075 1.27) (size 1 0.8) (layers "F.Cu" "F.Paste" "F.Mask") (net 6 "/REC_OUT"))
  (pad "4" smd rect (at 3.075 -1.27) (size 1 0.8) (layers "F.Cu" "F.Paste" "F.Mask") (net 3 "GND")))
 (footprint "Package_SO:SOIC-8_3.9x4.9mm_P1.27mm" (layer "F.Cu") (at 117 100)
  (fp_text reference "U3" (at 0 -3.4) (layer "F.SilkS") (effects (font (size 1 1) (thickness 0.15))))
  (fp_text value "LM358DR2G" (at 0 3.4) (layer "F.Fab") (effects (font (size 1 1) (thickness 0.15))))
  (pad "1" smd roundrect (at -2.475 -1.905) (size 1.95 0.6) (layers "F.Cu" "F.Paste" "F.Mask") (roundrect_rratio 0.25) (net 52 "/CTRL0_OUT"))
  (pad "2" smd roundrect (at -2.475 -0.635) (size 1.95 0.6) (layers "F.Cu" "F.Paste" "F.Mask") (roundrect_rratio 0.25) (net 51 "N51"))
  (pad "3" smd roundrect (at -2.475 0.635) (size 1.95 0.6) (layers "F.Cu" "F.Paste" "F.Mask") (roundrect_rratio 0.25) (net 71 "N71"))
  (pad "4" smd roundrect (at -2.475 1.905) (size 1.95 0.6) (layers "F.Cu" "F.Paste" "F.Mask") (roundrect_rratio 0.25) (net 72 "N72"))
  (pad "5" smd roundrect (at 2.475 1.905) (size 1.95 0.6) (layers "F.Cu" "F.Paste" "F.Mask") (roundrect_rratio 0.25) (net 59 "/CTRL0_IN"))
  (pad "6" smd roundrect (at 2.475 0.635) (size 1.95 0.6) (layers "F.Cu" "F.Paste" "F.Mask") (roundrect_rratio 0.25) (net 56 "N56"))
  (pad "7" smd roundrect (at 2.475 -0.635) (size 1.95 0.6) (layers "F.Cu" "F.Paste" "F.Mask") (roundrect_rratio 0.25) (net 56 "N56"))
  (pad "8" smd roundrect (at 2.475 -1.905) (size 1.95 0.6) (layers "F.Cu" "F.Paste" "F.Mask") (roundrect_rratio 0.25) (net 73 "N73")))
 (gr_rect (start 83 86) (end 123 116) (layer "Edge.Cuts") (width 0.1) (fill none))
 (segment (start 90 98) (end 90 91.888027) (width 0.2) (layer "F.Cu") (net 1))
 (segment (start 89.45 98.55) (end 90 98) (width 0.2) (layer "F.Cu") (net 1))
 (segment (start 92.138027 89.75) (end 92.55 89.75) (width 0.2) (layer "F.Cu") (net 1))
 (segment (start 88.625 98.55) (end 89.45 98.55) (width 0.2) (layer "F.Cu") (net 1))
 (segment (start 90 91.888027) (end 92.138027 89.75) (width 0.2) (layer "F.Cu") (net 1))
 (segment (start 86.25 112) (end 84.40048 110.15048) (width 0.4) (layer "F.Cu") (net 53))
 (segment (start 84.40048 107.25452) (end 86.925 104.73) (width 0.4) (layer "F.Cu") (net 53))
 (segment (start 84.40048 110.15048) (end 84.40048 107.25452) (width 0.4) (layer "F.Cu") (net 53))
 (segment (start 85 109) (end 85 108) (width 0.4) (layer "F.Cu") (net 54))
 (segment (start 88.25 109) (end 85 109) (width 0.4) (layer "F.Cu") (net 54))
 (segment (start 91.25 112) (end 88.25 109) (width 0.4) (layer "F.Cu") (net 54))
 (segment (start 85.73 107.27) (end 86.925 107.27) (width 0.4) (layer "F.Cu") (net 54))
 (segment (start 85 108) (end 85.73 107.27) (width 0.4) (layer "F.Cu") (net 54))
 (segment (start 96.75 87.75) (end 96 87) (width 0.2) (layer "F.Cu") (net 45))
 (segment (start 96 87) (end 94.6 87) (width 0.2) (layer "F.Cu") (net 45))
 (segment (start 96.75 88.55) (end 96.75 87.75) (width 0.2) (layer "F.Cu") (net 45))
 (segment (start 97.25 88.55) (end 97.25 87.95) (width 0.2) (layer "F.Cu") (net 44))
 (segment (start 97.25 87.95) (end 98.2 87) (width 0.2) (layer "F.Cu") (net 44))
 (segment (start 110.24952 95.068803) (end 110.24952 95.741197) (width 0.2) (layer "F.Cu") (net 31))
 (segment (start 108.975 94.135) (end 109.315717 94.135) (width 0.2) (layer "F.Cu") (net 31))
 (segment (start 99.87 93.75) (end 99.45 93.75) (width 0.2) (layer "F.Cu") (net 31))
 (segment (start 110.24952 95.741197) (end 109.986197 96.00452) (width 0.2) (layer "F.Cu") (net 31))
 (segment (start 109.986197 96.00452) (end 102.116493 96.00452) (width 0.2) (layer "F.Cu") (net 31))
 (segment (start 102.116493 96.00452) (end 99.861973 93.75) (width 0.2) (layer "F.Cu") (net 31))
 (segment (start 109.315717 94.135) (end 110.24952 95.068803) (width 0.2) (layer "F.Cu") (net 31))
 (segment (start 99.861973 93.75) (end 99.45 93.75) (width 0.2) (layer "F.Cu") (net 31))
 (segment (start 103.013803 92.26548) (end 101.998323 91.25) (width 0.2) (layer "F.Cu") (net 36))
 (segment (start 108.37548 92.26548) (end 103.013803 92.26548) (width 0.2) (layer "F.Cu") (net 36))
 (segment (start 101.998323 91.25) (end 99.45 91.25) (width 0.2) (layer "F.Cu") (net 36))
 (segment (start 108.975 92.865) (end 108.37548 92.26548) (width 0.2) (layer "F.Cu") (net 36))
 (segment (start 103.18 90.75) (end 99.45 90.75) (width 0.2) (layer "F.Cu") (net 37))
 (segment (start 104.025 91.595) (end 103.18 90.75) (width 0.2) (layer "F.Cu") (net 37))
 (segment (start 100.014015 91.75) (end 99.45 91.75) (width 0.2) (layer "F.Cu") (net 35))
 (segment (start 104.025 92.865) (end 101.129015 92.865) (width 0.2) (layer "F.Cu") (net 35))
 (segment (start 101.129015 92.865) (end 100.014015 91.75) (width 0.2) (layer "F.Cu") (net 35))
 (segment (start 101.834022 94.135) (end 99.949022 92.25) (width 0.2) (layer "F.Cu") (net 34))
 (segment (start 99.949022 92.25) (end 99.45 92.25) (width 0.2) (layer "F.Cu") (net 34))
 (segment (start 104.025 94.135) (end 101.834022 94.135) (width 0.2) (layer "F.Cu") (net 34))
 (segment (start 101.917453 94.80548) (end 99.861973 92.75) (width 0.2) (layer "F.Cu") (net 33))
 (segment (start 108.975 95.405) (end 108.37548 94.80548) (width 0.2) (layer "F.Cu") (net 33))
 (segment (start 108.37548 94.80548) (end 101.917453 94.80548) (width 0.2) (layer "F.Cu") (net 33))
 (segment (start 99.861973 92.75) (end 99.45 92.75) (width 0.2) (layer "F.Cu") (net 33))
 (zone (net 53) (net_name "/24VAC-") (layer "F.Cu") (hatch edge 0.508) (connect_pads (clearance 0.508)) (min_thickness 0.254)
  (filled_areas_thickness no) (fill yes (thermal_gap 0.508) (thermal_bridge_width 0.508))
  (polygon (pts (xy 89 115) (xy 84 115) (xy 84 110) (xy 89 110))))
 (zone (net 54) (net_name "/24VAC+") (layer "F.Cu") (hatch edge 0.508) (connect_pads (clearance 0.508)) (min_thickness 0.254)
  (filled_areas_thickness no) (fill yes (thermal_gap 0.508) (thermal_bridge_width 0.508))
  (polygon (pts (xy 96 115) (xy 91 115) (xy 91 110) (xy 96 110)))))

